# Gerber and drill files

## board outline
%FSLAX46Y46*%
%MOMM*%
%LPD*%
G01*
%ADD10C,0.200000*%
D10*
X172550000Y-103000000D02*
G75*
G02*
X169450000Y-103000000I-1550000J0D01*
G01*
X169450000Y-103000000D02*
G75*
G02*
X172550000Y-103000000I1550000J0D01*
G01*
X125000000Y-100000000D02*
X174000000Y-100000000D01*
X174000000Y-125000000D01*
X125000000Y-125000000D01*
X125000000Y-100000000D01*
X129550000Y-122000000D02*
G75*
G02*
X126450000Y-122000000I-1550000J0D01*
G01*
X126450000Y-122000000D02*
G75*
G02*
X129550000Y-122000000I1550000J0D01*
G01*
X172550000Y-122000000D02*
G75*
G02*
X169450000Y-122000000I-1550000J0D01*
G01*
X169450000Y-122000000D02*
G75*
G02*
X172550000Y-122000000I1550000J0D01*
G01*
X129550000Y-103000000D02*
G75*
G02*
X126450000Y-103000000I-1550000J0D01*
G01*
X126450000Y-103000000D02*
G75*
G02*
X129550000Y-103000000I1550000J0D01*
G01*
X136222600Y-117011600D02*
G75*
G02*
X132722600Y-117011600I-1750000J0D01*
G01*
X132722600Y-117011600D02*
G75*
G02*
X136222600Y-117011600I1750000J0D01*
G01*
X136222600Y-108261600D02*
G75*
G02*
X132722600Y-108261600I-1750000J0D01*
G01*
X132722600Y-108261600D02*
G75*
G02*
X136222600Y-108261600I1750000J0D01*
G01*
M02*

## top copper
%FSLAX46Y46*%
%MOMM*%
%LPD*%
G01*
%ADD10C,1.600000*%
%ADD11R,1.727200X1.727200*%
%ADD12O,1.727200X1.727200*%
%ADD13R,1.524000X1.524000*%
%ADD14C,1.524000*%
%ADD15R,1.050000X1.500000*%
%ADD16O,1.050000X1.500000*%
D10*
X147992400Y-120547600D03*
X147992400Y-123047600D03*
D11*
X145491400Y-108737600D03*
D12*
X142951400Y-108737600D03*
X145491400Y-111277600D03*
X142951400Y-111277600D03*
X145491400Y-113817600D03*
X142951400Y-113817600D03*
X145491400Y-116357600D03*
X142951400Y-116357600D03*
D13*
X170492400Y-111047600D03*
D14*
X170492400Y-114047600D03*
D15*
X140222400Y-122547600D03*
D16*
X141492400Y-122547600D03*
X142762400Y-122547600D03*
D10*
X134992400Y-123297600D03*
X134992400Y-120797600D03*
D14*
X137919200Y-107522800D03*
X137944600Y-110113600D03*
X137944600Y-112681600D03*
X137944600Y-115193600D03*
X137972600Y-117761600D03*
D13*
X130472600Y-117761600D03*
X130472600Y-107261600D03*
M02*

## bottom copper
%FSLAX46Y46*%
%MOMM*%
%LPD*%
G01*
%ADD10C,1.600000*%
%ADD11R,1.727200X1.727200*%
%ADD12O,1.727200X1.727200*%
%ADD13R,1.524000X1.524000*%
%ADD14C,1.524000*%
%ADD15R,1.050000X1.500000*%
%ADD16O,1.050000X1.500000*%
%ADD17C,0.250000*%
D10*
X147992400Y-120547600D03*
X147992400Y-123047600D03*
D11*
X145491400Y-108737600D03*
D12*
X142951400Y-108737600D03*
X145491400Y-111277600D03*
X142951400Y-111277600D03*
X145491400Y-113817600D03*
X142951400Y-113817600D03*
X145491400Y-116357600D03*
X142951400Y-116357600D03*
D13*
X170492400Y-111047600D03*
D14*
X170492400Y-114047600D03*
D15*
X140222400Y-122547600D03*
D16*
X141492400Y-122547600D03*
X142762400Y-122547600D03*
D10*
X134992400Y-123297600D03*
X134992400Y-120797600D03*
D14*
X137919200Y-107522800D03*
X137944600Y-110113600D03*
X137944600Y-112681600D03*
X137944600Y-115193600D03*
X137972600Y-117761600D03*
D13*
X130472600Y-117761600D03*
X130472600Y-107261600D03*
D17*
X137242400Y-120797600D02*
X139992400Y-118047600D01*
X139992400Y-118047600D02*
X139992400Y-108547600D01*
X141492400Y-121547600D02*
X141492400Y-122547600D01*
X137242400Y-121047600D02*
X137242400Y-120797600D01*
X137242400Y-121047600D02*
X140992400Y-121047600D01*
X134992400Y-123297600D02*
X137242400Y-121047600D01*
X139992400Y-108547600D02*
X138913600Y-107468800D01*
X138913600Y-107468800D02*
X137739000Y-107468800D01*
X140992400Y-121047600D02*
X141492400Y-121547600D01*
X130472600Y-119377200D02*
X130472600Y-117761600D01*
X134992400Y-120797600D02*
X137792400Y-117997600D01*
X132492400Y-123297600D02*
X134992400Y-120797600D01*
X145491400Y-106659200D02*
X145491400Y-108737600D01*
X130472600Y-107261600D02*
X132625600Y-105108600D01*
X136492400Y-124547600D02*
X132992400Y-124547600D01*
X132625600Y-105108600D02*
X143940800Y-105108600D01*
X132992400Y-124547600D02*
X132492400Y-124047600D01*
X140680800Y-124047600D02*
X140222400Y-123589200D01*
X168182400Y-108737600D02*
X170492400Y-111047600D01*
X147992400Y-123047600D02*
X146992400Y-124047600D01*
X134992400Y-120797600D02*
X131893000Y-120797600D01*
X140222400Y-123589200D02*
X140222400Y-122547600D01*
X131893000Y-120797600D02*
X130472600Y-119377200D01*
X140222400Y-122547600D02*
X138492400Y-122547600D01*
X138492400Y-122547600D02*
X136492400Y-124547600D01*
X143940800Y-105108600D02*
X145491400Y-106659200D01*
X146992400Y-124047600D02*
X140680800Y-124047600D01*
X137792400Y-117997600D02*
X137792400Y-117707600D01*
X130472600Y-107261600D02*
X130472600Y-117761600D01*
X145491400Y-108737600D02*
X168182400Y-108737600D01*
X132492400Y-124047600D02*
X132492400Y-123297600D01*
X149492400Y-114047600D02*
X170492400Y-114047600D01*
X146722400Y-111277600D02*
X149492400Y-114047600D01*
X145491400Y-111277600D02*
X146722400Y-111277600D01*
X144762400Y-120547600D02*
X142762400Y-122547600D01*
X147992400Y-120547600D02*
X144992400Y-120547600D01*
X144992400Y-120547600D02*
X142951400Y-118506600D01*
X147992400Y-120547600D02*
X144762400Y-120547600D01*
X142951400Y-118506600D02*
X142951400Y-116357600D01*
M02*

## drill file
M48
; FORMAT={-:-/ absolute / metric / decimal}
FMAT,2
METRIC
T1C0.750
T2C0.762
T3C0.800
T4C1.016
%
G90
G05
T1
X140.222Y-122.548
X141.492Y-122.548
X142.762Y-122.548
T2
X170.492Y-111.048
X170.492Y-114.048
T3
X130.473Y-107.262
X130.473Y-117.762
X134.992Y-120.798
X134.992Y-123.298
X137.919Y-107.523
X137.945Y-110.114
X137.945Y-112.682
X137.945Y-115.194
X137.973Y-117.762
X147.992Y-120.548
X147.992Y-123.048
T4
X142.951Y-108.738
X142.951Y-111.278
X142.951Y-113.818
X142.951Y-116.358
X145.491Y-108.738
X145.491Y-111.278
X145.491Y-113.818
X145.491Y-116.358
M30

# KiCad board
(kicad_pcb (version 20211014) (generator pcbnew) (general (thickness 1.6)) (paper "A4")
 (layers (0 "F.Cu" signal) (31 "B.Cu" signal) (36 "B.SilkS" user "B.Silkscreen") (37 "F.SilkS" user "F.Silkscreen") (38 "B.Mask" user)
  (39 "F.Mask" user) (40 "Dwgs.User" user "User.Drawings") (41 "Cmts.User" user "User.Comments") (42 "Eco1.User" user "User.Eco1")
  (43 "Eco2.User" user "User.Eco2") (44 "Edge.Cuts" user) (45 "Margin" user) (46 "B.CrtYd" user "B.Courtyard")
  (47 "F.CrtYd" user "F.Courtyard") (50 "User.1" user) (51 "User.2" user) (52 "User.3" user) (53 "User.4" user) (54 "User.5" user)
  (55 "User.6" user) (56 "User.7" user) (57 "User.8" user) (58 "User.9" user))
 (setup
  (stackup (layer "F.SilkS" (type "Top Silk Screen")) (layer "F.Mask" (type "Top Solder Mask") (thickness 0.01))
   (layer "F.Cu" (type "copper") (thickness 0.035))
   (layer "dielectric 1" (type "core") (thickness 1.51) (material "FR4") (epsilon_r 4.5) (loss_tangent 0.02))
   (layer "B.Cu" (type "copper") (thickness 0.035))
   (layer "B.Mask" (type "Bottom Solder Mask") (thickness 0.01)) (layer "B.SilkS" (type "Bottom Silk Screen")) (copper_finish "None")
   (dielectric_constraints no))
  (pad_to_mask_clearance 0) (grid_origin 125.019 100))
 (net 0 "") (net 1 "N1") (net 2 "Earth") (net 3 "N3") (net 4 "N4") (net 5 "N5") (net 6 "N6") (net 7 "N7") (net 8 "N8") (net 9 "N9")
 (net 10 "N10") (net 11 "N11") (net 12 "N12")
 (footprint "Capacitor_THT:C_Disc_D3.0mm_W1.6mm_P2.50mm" (layer "F.Cu") (at 147.9924 120.5476 -90)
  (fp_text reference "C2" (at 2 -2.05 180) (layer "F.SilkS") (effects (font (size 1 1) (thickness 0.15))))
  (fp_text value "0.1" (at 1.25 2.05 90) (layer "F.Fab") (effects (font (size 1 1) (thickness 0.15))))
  (pad "1" thru_hole circle (at 0 0 270) (size 1.6 1.6) (drill 0.8) (layers *.Cu *.Mask) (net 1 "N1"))
  (pad "2" thru_hole circle (at 2.5 0 270) (size 1.6 1.6) (drill 0.8) (layers *.Cu *.Mask) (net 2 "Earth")))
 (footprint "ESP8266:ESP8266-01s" (layer "F.Cu") (at 142.9514 108.7376)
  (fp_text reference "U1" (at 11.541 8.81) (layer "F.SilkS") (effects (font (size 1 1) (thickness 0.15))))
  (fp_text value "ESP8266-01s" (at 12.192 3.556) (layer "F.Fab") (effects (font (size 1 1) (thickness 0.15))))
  (pad "1" thru_hole rect (at 2.54 0) (size 1.7272 1.7272) (drill 1.016) (layers *.Cu *.Mask) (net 2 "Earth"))
  (pad "2" thru_hole oval (at 0 0) (size 1.7272 1.7272) (drill 1.016) (layers *.Cu *.Mask) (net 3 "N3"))
  (pad "3" thru_hole oval (at 2.54 2.54) (size 1.7272 1.7272) (drill 1.016) (layers *.Cu *.Mask) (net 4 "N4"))
  (pad "4" thru_hole oval (at 0 2.54) (size 1.7272 1.7272) (drill 1.016) (layers *.Cu *.Mask) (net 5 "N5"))
  (pad "5" thru_hole oval (at 2.54 5.08) (size 1.7272 1.7272) (drill 1.016) (layers *.Cu *.Mask) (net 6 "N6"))
  (pad "6" thru_hole oval (at 0 5.08) (size 1.7272 1.7272) (drill 1.016) (layers *.Cu *.Mask) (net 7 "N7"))
  (pad "7" thru_hole oval (at 2.54 7.62) (size 1.7272 1.7272) (drill 1.016) (layers *.Cu *.Mask) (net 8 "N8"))
  (pad "8" thru_hole oval (at 0 7.62) (size 1.7272 1.7272) (drill 1.016) (layers *.Cu *.Mask) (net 1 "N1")))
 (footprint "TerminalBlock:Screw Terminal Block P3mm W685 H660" (layer "F.Cu") (at 170.4924 111.0476 -90)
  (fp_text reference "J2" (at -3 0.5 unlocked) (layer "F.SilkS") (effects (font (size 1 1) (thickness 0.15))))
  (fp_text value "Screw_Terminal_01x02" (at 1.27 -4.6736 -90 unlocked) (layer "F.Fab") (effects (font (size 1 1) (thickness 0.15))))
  (pad "1" thru_hole rect (at 0 0 270) (size 1.524 1.524) (drill 0.762) (layers *.Cu *.Mask) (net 2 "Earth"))
  (pad "2" thru_hole circle (at 3 0 270) (size 1.524 1.524) (drill 0.762) (layers *.Cu *.Mask) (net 4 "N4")))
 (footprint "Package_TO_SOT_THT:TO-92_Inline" (layer "F.Cu") (at 140.2224 122.5476)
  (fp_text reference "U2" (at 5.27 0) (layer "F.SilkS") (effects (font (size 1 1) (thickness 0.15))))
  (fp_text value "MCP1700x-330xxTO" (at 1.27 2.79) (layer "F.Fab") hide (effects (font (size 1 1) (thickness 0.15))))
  (pad "1" thru_hole rect (at 0 0) (size 1.05 1.5) (drill 0.75) (layers *.Cu *.Mask) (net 2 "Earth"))
  (pad "2" thru_hole oval (at 1.27 0) (size 1.05 1.5) (drill 0.75) (layers *.Cu *.Mask) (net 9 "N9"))
  (pad "3" thru_hole oval (at 2.54 0) (size 1.05 1.5) (drill 0.75) (layers *.Cu *.Mask) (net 1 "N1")))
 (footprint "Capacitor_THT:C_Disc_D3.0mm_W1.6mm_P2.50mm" (layer "F.Cu") (at 134.9924 123.2976 90)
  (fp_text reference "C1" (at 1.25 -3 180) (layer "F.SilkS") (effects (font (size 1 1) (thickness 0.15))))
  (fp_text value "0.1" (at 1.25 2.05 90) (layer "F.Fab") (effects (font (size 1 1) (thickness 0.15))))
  (pad "1" thru_hole circle (at 0 0 90) (size 1.6 1.6) (drill 0.8) (layers *.Cu *.Mask) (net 9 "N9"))
  (pad "2" thru_hole circle (at 2.5 0 90) (size 1.6 1.6) (drill 0.8) (layers *.Cu *.Mask) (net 2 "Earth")))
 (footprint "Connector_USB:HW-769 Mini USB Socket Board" (layer "F.Cu") (at 139.7226 119.5116)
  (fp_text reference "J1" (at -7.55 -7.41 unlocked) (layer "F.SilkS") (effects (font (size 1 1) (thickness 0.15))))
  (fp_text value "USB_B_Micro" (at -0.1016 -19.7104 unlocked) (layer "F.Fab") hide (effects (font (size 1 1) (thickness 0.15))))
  (fp_circle (center -5.25 -2.5) (end -3.5 -2.5) (layer "Edge.Cuts") (width 0.2) (fill none))
  (fp_circle (center -5.25 -11.25) (end -3.5 -11.25) (layer "Edge.Cuts") (width 0.2) (fill none))
  (pad "1" thru_hole circle (at -1.8034 -11.9888) (size 1.524 1.524) (drill 0.8) (layers *.Cu *.Mask) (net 9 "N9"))
  (pad "2" thru_hole circle (at -1.778 -9.398) (size 1.524 1.524) (drill 0.8) (layers *.Cu *.Mask) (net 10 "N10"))
  (pad "3" thru_hole circle (at -1.778 -6.83) (size 1.524 1.524) (drill 0.8) (layers *.Cu *.Mask) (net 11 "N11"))
  (pad "4" thru_hole circle (at -1.778 -4.318) (size 1.524 1.524) (drill 0.8) (layers *.Cu *.Mask) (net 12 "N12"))
  (pad "5" thru_hole circle (at -1.75 -1.75) (size 1.524 1.524) (drill 0.8) (layers *.Cu *.Mask) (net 2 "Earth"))
  (pad "6" thru_hole rect (at -9.25 -1.75) (size 1.524 1.524) (drill 0.8) (layers *.Cu *.Mask) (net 2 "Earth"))
  (pad "7" thru_hole rect (at -9.25 -12.25) (size 1.524 1.524) (drill 0.8) (layers *.Cu *.Mask) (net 2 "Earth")))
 (gr_circle (center 171 103) (end 172.55 103) (layer "Edge.Cuts") (width 0.2) (fill none))
 (gr_rect (start 125 100) (end 174 125) (layer "Edge.Cuts") (width 0.2) (fill none))
 (gr_circle (center 128 122) (end 129.55 122) (layer "Edge.Cuts") (width 0.2) (fill none))
 (gr_circle (center 171 122) (end 172.55 122) (layer "Edge.Cuts") (width 0.2) (fill none))
 (gr_circle (center 128 103) (end 129.55 103) (layer "Edge.Cuts") (width 0.2) (fill none))
 (segment (start 137.2424 120.7976) (end 139.9924 118.0476) (width 0.25) (layer "B.Cu") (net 9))
 (segment (start 139.9924 118.0476) (end 139.9924 108.5476) (width 0.25) (layer "B.Cu") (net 9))
 (segment (start 141.4924 121.5476) (end 141.4924 122.5476) (width 0.25) (layer "B.Cu") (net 9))
 (segment (start 137.2424 121.0476) (end 137.2424 120.7976) (width 0.25) (layer "B.Cu") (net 9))
 (segment (start 137.2424 121.0476) (end 140.9924 121.0476) (width 0.25) (layer "B.Cu") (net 9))
 (segment (start 134.9924 123.2976) (end 137.2424 121.0476) (width 0.25) (layer "B.Cu") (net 9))
 (segment (start 139.9924 108.5476) (end 138.9136 107.4688) (width 0.25) (layer "B.Cu") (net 9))
 (segment (start 138.9136 107.4688) (end 137.739 107.4688) (width 0.25) (layer "B.Cu") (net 9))
 (segment (start 140.9924 121.0476) (end 141.4924 121.5476) (width 0.25) (layer "B.Cu") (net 9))
 (segment (start 130.4726 119.3772) (end 130.4726 117.7616) (width 0.25) (layer "B.Cu") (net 2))
 (segment (start 134.9924 120.7976) (end 137.7924 117.9976) (width 0.25) (layer "B.Cu") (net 2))
 (segment (start 132.4924 123.2976) (end 134.9924 120.7976) (width 0.25) (layer "B.Cu") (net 2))
 (segment (start 145.4914 106.6592) (end 145.4914 108.7376) (width 0.25) (layer "B.Cu") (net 2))
 (segment (start 130.4726 107.2616) (end 132.6256 105.1086) (width 0.25) (layer "B.Cu") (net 2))
 (segment (start 136.4924 124.5476) (end 132.9924 124.5476) (width 0.25) (layer "B.Cu") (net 2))
 (segment (start 132.6256 105.1086) (end 143.9408 105.1086) (width 0.25) (layer "B.Cu") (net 2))
 (segment (start 132.9924 124.5476) (end 132.4924 124.0476) (width 0.25) (layer "B.Cu") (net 2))
 (segment (start 140.6808 124.0476) (end 140.2224 123.5892) (width 0.25) (layer "B.Cu") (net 2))
 (segment (start 168.1824 108.7376) (end 170.4924 111.0476) (width 0.25) (layer "B.Cu") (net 2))
 (segment (start 147.9924 123.0476) (end 146.9924 124.0476) (width 0.25) (layer "B.Cu") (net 2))
 (segment (start 134.9924 120.7976) (end 131.893 120.7976) (width 0.25) (layer "B.Cu") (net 2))
 (segment (start 140.2224 123.5892) (end 140.2224 122.5476) (width 0.25) (layer "B.Cu") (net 2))
 (segment (start 131.893 120.7976) (end 130.4726 119.3772) (width 0.25) (layer "B.Cu") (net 2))
 (segment (start 140.2224 122.5476) (end 138.4924 122.5476) (width 0.25) (layer "B.Cu") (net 2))
 (segment (start 138.4924 122.5476) (end 136.4924 124.5476) (width 0.25) (layer "B.Cu") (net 2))
 (segment (start 143.9408 105.1086) (end 145.4914 106.6592) (width 0.25) (layer "B.Cu") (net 2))
 (segment (start 146.9924 124.0476) (end 140.6808 124.0476) (width 0.25) (layer "B.Cu") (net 2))
 (segment (start 137.7924 117.9976) (end 137.7924 117.7076) (width 0.25) (layer "B.Cu") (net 2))
 (segment (start 130.4726 107.2616) (end 130.4726 117.7616) (width 0.25) (layer "B.Cu") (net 2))
 (segment (start 145.4914 108.7376) (end 168.1824 108.7376) (width 0.25) (layer "B.Cu") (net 2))
 (segment (start 132.4924 124.0476) (end 132.4924 123.2976) (width 0.25) (layer "B.Cu") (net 2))
 (segment (start 149.4924 114.0476) (end 170.4924 114.0476) (width 0.25) (layer "B.Cu") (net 4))
 (segment (start 146.7224 111.2776) (end 149.4924 114.0476) (width 0.25) (layer "B.Cu") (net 4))
 (segment (start 145.4914 111.2776) (end 146.7224 111.2776) (width 0.25) (layer "B.Cu") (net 4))
 (segment (start 144.7624 120.5476) (end 142.7624 122.5476) (width 0.25) (layer "B.Cu") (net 1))
 (segment (start 147.9924 120.5476) (end 144.9924 120.5476) (width 0.25) (layer "B.Cu") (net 1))
 (segment (start 144.9924 120.5476) (end 142.9514 118.5066) (width 0.25) (layer "B.Cu") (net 1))
 (segment (start 147.9924 120.5476) (end 144.7624 120.5476) (width 0.25) (layer "B.Cu") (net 1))
 (segment (start 142.9514 118.5066) (end 142.9514 116.3576) (width 0.25) (layer "B.Cu") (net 1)))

